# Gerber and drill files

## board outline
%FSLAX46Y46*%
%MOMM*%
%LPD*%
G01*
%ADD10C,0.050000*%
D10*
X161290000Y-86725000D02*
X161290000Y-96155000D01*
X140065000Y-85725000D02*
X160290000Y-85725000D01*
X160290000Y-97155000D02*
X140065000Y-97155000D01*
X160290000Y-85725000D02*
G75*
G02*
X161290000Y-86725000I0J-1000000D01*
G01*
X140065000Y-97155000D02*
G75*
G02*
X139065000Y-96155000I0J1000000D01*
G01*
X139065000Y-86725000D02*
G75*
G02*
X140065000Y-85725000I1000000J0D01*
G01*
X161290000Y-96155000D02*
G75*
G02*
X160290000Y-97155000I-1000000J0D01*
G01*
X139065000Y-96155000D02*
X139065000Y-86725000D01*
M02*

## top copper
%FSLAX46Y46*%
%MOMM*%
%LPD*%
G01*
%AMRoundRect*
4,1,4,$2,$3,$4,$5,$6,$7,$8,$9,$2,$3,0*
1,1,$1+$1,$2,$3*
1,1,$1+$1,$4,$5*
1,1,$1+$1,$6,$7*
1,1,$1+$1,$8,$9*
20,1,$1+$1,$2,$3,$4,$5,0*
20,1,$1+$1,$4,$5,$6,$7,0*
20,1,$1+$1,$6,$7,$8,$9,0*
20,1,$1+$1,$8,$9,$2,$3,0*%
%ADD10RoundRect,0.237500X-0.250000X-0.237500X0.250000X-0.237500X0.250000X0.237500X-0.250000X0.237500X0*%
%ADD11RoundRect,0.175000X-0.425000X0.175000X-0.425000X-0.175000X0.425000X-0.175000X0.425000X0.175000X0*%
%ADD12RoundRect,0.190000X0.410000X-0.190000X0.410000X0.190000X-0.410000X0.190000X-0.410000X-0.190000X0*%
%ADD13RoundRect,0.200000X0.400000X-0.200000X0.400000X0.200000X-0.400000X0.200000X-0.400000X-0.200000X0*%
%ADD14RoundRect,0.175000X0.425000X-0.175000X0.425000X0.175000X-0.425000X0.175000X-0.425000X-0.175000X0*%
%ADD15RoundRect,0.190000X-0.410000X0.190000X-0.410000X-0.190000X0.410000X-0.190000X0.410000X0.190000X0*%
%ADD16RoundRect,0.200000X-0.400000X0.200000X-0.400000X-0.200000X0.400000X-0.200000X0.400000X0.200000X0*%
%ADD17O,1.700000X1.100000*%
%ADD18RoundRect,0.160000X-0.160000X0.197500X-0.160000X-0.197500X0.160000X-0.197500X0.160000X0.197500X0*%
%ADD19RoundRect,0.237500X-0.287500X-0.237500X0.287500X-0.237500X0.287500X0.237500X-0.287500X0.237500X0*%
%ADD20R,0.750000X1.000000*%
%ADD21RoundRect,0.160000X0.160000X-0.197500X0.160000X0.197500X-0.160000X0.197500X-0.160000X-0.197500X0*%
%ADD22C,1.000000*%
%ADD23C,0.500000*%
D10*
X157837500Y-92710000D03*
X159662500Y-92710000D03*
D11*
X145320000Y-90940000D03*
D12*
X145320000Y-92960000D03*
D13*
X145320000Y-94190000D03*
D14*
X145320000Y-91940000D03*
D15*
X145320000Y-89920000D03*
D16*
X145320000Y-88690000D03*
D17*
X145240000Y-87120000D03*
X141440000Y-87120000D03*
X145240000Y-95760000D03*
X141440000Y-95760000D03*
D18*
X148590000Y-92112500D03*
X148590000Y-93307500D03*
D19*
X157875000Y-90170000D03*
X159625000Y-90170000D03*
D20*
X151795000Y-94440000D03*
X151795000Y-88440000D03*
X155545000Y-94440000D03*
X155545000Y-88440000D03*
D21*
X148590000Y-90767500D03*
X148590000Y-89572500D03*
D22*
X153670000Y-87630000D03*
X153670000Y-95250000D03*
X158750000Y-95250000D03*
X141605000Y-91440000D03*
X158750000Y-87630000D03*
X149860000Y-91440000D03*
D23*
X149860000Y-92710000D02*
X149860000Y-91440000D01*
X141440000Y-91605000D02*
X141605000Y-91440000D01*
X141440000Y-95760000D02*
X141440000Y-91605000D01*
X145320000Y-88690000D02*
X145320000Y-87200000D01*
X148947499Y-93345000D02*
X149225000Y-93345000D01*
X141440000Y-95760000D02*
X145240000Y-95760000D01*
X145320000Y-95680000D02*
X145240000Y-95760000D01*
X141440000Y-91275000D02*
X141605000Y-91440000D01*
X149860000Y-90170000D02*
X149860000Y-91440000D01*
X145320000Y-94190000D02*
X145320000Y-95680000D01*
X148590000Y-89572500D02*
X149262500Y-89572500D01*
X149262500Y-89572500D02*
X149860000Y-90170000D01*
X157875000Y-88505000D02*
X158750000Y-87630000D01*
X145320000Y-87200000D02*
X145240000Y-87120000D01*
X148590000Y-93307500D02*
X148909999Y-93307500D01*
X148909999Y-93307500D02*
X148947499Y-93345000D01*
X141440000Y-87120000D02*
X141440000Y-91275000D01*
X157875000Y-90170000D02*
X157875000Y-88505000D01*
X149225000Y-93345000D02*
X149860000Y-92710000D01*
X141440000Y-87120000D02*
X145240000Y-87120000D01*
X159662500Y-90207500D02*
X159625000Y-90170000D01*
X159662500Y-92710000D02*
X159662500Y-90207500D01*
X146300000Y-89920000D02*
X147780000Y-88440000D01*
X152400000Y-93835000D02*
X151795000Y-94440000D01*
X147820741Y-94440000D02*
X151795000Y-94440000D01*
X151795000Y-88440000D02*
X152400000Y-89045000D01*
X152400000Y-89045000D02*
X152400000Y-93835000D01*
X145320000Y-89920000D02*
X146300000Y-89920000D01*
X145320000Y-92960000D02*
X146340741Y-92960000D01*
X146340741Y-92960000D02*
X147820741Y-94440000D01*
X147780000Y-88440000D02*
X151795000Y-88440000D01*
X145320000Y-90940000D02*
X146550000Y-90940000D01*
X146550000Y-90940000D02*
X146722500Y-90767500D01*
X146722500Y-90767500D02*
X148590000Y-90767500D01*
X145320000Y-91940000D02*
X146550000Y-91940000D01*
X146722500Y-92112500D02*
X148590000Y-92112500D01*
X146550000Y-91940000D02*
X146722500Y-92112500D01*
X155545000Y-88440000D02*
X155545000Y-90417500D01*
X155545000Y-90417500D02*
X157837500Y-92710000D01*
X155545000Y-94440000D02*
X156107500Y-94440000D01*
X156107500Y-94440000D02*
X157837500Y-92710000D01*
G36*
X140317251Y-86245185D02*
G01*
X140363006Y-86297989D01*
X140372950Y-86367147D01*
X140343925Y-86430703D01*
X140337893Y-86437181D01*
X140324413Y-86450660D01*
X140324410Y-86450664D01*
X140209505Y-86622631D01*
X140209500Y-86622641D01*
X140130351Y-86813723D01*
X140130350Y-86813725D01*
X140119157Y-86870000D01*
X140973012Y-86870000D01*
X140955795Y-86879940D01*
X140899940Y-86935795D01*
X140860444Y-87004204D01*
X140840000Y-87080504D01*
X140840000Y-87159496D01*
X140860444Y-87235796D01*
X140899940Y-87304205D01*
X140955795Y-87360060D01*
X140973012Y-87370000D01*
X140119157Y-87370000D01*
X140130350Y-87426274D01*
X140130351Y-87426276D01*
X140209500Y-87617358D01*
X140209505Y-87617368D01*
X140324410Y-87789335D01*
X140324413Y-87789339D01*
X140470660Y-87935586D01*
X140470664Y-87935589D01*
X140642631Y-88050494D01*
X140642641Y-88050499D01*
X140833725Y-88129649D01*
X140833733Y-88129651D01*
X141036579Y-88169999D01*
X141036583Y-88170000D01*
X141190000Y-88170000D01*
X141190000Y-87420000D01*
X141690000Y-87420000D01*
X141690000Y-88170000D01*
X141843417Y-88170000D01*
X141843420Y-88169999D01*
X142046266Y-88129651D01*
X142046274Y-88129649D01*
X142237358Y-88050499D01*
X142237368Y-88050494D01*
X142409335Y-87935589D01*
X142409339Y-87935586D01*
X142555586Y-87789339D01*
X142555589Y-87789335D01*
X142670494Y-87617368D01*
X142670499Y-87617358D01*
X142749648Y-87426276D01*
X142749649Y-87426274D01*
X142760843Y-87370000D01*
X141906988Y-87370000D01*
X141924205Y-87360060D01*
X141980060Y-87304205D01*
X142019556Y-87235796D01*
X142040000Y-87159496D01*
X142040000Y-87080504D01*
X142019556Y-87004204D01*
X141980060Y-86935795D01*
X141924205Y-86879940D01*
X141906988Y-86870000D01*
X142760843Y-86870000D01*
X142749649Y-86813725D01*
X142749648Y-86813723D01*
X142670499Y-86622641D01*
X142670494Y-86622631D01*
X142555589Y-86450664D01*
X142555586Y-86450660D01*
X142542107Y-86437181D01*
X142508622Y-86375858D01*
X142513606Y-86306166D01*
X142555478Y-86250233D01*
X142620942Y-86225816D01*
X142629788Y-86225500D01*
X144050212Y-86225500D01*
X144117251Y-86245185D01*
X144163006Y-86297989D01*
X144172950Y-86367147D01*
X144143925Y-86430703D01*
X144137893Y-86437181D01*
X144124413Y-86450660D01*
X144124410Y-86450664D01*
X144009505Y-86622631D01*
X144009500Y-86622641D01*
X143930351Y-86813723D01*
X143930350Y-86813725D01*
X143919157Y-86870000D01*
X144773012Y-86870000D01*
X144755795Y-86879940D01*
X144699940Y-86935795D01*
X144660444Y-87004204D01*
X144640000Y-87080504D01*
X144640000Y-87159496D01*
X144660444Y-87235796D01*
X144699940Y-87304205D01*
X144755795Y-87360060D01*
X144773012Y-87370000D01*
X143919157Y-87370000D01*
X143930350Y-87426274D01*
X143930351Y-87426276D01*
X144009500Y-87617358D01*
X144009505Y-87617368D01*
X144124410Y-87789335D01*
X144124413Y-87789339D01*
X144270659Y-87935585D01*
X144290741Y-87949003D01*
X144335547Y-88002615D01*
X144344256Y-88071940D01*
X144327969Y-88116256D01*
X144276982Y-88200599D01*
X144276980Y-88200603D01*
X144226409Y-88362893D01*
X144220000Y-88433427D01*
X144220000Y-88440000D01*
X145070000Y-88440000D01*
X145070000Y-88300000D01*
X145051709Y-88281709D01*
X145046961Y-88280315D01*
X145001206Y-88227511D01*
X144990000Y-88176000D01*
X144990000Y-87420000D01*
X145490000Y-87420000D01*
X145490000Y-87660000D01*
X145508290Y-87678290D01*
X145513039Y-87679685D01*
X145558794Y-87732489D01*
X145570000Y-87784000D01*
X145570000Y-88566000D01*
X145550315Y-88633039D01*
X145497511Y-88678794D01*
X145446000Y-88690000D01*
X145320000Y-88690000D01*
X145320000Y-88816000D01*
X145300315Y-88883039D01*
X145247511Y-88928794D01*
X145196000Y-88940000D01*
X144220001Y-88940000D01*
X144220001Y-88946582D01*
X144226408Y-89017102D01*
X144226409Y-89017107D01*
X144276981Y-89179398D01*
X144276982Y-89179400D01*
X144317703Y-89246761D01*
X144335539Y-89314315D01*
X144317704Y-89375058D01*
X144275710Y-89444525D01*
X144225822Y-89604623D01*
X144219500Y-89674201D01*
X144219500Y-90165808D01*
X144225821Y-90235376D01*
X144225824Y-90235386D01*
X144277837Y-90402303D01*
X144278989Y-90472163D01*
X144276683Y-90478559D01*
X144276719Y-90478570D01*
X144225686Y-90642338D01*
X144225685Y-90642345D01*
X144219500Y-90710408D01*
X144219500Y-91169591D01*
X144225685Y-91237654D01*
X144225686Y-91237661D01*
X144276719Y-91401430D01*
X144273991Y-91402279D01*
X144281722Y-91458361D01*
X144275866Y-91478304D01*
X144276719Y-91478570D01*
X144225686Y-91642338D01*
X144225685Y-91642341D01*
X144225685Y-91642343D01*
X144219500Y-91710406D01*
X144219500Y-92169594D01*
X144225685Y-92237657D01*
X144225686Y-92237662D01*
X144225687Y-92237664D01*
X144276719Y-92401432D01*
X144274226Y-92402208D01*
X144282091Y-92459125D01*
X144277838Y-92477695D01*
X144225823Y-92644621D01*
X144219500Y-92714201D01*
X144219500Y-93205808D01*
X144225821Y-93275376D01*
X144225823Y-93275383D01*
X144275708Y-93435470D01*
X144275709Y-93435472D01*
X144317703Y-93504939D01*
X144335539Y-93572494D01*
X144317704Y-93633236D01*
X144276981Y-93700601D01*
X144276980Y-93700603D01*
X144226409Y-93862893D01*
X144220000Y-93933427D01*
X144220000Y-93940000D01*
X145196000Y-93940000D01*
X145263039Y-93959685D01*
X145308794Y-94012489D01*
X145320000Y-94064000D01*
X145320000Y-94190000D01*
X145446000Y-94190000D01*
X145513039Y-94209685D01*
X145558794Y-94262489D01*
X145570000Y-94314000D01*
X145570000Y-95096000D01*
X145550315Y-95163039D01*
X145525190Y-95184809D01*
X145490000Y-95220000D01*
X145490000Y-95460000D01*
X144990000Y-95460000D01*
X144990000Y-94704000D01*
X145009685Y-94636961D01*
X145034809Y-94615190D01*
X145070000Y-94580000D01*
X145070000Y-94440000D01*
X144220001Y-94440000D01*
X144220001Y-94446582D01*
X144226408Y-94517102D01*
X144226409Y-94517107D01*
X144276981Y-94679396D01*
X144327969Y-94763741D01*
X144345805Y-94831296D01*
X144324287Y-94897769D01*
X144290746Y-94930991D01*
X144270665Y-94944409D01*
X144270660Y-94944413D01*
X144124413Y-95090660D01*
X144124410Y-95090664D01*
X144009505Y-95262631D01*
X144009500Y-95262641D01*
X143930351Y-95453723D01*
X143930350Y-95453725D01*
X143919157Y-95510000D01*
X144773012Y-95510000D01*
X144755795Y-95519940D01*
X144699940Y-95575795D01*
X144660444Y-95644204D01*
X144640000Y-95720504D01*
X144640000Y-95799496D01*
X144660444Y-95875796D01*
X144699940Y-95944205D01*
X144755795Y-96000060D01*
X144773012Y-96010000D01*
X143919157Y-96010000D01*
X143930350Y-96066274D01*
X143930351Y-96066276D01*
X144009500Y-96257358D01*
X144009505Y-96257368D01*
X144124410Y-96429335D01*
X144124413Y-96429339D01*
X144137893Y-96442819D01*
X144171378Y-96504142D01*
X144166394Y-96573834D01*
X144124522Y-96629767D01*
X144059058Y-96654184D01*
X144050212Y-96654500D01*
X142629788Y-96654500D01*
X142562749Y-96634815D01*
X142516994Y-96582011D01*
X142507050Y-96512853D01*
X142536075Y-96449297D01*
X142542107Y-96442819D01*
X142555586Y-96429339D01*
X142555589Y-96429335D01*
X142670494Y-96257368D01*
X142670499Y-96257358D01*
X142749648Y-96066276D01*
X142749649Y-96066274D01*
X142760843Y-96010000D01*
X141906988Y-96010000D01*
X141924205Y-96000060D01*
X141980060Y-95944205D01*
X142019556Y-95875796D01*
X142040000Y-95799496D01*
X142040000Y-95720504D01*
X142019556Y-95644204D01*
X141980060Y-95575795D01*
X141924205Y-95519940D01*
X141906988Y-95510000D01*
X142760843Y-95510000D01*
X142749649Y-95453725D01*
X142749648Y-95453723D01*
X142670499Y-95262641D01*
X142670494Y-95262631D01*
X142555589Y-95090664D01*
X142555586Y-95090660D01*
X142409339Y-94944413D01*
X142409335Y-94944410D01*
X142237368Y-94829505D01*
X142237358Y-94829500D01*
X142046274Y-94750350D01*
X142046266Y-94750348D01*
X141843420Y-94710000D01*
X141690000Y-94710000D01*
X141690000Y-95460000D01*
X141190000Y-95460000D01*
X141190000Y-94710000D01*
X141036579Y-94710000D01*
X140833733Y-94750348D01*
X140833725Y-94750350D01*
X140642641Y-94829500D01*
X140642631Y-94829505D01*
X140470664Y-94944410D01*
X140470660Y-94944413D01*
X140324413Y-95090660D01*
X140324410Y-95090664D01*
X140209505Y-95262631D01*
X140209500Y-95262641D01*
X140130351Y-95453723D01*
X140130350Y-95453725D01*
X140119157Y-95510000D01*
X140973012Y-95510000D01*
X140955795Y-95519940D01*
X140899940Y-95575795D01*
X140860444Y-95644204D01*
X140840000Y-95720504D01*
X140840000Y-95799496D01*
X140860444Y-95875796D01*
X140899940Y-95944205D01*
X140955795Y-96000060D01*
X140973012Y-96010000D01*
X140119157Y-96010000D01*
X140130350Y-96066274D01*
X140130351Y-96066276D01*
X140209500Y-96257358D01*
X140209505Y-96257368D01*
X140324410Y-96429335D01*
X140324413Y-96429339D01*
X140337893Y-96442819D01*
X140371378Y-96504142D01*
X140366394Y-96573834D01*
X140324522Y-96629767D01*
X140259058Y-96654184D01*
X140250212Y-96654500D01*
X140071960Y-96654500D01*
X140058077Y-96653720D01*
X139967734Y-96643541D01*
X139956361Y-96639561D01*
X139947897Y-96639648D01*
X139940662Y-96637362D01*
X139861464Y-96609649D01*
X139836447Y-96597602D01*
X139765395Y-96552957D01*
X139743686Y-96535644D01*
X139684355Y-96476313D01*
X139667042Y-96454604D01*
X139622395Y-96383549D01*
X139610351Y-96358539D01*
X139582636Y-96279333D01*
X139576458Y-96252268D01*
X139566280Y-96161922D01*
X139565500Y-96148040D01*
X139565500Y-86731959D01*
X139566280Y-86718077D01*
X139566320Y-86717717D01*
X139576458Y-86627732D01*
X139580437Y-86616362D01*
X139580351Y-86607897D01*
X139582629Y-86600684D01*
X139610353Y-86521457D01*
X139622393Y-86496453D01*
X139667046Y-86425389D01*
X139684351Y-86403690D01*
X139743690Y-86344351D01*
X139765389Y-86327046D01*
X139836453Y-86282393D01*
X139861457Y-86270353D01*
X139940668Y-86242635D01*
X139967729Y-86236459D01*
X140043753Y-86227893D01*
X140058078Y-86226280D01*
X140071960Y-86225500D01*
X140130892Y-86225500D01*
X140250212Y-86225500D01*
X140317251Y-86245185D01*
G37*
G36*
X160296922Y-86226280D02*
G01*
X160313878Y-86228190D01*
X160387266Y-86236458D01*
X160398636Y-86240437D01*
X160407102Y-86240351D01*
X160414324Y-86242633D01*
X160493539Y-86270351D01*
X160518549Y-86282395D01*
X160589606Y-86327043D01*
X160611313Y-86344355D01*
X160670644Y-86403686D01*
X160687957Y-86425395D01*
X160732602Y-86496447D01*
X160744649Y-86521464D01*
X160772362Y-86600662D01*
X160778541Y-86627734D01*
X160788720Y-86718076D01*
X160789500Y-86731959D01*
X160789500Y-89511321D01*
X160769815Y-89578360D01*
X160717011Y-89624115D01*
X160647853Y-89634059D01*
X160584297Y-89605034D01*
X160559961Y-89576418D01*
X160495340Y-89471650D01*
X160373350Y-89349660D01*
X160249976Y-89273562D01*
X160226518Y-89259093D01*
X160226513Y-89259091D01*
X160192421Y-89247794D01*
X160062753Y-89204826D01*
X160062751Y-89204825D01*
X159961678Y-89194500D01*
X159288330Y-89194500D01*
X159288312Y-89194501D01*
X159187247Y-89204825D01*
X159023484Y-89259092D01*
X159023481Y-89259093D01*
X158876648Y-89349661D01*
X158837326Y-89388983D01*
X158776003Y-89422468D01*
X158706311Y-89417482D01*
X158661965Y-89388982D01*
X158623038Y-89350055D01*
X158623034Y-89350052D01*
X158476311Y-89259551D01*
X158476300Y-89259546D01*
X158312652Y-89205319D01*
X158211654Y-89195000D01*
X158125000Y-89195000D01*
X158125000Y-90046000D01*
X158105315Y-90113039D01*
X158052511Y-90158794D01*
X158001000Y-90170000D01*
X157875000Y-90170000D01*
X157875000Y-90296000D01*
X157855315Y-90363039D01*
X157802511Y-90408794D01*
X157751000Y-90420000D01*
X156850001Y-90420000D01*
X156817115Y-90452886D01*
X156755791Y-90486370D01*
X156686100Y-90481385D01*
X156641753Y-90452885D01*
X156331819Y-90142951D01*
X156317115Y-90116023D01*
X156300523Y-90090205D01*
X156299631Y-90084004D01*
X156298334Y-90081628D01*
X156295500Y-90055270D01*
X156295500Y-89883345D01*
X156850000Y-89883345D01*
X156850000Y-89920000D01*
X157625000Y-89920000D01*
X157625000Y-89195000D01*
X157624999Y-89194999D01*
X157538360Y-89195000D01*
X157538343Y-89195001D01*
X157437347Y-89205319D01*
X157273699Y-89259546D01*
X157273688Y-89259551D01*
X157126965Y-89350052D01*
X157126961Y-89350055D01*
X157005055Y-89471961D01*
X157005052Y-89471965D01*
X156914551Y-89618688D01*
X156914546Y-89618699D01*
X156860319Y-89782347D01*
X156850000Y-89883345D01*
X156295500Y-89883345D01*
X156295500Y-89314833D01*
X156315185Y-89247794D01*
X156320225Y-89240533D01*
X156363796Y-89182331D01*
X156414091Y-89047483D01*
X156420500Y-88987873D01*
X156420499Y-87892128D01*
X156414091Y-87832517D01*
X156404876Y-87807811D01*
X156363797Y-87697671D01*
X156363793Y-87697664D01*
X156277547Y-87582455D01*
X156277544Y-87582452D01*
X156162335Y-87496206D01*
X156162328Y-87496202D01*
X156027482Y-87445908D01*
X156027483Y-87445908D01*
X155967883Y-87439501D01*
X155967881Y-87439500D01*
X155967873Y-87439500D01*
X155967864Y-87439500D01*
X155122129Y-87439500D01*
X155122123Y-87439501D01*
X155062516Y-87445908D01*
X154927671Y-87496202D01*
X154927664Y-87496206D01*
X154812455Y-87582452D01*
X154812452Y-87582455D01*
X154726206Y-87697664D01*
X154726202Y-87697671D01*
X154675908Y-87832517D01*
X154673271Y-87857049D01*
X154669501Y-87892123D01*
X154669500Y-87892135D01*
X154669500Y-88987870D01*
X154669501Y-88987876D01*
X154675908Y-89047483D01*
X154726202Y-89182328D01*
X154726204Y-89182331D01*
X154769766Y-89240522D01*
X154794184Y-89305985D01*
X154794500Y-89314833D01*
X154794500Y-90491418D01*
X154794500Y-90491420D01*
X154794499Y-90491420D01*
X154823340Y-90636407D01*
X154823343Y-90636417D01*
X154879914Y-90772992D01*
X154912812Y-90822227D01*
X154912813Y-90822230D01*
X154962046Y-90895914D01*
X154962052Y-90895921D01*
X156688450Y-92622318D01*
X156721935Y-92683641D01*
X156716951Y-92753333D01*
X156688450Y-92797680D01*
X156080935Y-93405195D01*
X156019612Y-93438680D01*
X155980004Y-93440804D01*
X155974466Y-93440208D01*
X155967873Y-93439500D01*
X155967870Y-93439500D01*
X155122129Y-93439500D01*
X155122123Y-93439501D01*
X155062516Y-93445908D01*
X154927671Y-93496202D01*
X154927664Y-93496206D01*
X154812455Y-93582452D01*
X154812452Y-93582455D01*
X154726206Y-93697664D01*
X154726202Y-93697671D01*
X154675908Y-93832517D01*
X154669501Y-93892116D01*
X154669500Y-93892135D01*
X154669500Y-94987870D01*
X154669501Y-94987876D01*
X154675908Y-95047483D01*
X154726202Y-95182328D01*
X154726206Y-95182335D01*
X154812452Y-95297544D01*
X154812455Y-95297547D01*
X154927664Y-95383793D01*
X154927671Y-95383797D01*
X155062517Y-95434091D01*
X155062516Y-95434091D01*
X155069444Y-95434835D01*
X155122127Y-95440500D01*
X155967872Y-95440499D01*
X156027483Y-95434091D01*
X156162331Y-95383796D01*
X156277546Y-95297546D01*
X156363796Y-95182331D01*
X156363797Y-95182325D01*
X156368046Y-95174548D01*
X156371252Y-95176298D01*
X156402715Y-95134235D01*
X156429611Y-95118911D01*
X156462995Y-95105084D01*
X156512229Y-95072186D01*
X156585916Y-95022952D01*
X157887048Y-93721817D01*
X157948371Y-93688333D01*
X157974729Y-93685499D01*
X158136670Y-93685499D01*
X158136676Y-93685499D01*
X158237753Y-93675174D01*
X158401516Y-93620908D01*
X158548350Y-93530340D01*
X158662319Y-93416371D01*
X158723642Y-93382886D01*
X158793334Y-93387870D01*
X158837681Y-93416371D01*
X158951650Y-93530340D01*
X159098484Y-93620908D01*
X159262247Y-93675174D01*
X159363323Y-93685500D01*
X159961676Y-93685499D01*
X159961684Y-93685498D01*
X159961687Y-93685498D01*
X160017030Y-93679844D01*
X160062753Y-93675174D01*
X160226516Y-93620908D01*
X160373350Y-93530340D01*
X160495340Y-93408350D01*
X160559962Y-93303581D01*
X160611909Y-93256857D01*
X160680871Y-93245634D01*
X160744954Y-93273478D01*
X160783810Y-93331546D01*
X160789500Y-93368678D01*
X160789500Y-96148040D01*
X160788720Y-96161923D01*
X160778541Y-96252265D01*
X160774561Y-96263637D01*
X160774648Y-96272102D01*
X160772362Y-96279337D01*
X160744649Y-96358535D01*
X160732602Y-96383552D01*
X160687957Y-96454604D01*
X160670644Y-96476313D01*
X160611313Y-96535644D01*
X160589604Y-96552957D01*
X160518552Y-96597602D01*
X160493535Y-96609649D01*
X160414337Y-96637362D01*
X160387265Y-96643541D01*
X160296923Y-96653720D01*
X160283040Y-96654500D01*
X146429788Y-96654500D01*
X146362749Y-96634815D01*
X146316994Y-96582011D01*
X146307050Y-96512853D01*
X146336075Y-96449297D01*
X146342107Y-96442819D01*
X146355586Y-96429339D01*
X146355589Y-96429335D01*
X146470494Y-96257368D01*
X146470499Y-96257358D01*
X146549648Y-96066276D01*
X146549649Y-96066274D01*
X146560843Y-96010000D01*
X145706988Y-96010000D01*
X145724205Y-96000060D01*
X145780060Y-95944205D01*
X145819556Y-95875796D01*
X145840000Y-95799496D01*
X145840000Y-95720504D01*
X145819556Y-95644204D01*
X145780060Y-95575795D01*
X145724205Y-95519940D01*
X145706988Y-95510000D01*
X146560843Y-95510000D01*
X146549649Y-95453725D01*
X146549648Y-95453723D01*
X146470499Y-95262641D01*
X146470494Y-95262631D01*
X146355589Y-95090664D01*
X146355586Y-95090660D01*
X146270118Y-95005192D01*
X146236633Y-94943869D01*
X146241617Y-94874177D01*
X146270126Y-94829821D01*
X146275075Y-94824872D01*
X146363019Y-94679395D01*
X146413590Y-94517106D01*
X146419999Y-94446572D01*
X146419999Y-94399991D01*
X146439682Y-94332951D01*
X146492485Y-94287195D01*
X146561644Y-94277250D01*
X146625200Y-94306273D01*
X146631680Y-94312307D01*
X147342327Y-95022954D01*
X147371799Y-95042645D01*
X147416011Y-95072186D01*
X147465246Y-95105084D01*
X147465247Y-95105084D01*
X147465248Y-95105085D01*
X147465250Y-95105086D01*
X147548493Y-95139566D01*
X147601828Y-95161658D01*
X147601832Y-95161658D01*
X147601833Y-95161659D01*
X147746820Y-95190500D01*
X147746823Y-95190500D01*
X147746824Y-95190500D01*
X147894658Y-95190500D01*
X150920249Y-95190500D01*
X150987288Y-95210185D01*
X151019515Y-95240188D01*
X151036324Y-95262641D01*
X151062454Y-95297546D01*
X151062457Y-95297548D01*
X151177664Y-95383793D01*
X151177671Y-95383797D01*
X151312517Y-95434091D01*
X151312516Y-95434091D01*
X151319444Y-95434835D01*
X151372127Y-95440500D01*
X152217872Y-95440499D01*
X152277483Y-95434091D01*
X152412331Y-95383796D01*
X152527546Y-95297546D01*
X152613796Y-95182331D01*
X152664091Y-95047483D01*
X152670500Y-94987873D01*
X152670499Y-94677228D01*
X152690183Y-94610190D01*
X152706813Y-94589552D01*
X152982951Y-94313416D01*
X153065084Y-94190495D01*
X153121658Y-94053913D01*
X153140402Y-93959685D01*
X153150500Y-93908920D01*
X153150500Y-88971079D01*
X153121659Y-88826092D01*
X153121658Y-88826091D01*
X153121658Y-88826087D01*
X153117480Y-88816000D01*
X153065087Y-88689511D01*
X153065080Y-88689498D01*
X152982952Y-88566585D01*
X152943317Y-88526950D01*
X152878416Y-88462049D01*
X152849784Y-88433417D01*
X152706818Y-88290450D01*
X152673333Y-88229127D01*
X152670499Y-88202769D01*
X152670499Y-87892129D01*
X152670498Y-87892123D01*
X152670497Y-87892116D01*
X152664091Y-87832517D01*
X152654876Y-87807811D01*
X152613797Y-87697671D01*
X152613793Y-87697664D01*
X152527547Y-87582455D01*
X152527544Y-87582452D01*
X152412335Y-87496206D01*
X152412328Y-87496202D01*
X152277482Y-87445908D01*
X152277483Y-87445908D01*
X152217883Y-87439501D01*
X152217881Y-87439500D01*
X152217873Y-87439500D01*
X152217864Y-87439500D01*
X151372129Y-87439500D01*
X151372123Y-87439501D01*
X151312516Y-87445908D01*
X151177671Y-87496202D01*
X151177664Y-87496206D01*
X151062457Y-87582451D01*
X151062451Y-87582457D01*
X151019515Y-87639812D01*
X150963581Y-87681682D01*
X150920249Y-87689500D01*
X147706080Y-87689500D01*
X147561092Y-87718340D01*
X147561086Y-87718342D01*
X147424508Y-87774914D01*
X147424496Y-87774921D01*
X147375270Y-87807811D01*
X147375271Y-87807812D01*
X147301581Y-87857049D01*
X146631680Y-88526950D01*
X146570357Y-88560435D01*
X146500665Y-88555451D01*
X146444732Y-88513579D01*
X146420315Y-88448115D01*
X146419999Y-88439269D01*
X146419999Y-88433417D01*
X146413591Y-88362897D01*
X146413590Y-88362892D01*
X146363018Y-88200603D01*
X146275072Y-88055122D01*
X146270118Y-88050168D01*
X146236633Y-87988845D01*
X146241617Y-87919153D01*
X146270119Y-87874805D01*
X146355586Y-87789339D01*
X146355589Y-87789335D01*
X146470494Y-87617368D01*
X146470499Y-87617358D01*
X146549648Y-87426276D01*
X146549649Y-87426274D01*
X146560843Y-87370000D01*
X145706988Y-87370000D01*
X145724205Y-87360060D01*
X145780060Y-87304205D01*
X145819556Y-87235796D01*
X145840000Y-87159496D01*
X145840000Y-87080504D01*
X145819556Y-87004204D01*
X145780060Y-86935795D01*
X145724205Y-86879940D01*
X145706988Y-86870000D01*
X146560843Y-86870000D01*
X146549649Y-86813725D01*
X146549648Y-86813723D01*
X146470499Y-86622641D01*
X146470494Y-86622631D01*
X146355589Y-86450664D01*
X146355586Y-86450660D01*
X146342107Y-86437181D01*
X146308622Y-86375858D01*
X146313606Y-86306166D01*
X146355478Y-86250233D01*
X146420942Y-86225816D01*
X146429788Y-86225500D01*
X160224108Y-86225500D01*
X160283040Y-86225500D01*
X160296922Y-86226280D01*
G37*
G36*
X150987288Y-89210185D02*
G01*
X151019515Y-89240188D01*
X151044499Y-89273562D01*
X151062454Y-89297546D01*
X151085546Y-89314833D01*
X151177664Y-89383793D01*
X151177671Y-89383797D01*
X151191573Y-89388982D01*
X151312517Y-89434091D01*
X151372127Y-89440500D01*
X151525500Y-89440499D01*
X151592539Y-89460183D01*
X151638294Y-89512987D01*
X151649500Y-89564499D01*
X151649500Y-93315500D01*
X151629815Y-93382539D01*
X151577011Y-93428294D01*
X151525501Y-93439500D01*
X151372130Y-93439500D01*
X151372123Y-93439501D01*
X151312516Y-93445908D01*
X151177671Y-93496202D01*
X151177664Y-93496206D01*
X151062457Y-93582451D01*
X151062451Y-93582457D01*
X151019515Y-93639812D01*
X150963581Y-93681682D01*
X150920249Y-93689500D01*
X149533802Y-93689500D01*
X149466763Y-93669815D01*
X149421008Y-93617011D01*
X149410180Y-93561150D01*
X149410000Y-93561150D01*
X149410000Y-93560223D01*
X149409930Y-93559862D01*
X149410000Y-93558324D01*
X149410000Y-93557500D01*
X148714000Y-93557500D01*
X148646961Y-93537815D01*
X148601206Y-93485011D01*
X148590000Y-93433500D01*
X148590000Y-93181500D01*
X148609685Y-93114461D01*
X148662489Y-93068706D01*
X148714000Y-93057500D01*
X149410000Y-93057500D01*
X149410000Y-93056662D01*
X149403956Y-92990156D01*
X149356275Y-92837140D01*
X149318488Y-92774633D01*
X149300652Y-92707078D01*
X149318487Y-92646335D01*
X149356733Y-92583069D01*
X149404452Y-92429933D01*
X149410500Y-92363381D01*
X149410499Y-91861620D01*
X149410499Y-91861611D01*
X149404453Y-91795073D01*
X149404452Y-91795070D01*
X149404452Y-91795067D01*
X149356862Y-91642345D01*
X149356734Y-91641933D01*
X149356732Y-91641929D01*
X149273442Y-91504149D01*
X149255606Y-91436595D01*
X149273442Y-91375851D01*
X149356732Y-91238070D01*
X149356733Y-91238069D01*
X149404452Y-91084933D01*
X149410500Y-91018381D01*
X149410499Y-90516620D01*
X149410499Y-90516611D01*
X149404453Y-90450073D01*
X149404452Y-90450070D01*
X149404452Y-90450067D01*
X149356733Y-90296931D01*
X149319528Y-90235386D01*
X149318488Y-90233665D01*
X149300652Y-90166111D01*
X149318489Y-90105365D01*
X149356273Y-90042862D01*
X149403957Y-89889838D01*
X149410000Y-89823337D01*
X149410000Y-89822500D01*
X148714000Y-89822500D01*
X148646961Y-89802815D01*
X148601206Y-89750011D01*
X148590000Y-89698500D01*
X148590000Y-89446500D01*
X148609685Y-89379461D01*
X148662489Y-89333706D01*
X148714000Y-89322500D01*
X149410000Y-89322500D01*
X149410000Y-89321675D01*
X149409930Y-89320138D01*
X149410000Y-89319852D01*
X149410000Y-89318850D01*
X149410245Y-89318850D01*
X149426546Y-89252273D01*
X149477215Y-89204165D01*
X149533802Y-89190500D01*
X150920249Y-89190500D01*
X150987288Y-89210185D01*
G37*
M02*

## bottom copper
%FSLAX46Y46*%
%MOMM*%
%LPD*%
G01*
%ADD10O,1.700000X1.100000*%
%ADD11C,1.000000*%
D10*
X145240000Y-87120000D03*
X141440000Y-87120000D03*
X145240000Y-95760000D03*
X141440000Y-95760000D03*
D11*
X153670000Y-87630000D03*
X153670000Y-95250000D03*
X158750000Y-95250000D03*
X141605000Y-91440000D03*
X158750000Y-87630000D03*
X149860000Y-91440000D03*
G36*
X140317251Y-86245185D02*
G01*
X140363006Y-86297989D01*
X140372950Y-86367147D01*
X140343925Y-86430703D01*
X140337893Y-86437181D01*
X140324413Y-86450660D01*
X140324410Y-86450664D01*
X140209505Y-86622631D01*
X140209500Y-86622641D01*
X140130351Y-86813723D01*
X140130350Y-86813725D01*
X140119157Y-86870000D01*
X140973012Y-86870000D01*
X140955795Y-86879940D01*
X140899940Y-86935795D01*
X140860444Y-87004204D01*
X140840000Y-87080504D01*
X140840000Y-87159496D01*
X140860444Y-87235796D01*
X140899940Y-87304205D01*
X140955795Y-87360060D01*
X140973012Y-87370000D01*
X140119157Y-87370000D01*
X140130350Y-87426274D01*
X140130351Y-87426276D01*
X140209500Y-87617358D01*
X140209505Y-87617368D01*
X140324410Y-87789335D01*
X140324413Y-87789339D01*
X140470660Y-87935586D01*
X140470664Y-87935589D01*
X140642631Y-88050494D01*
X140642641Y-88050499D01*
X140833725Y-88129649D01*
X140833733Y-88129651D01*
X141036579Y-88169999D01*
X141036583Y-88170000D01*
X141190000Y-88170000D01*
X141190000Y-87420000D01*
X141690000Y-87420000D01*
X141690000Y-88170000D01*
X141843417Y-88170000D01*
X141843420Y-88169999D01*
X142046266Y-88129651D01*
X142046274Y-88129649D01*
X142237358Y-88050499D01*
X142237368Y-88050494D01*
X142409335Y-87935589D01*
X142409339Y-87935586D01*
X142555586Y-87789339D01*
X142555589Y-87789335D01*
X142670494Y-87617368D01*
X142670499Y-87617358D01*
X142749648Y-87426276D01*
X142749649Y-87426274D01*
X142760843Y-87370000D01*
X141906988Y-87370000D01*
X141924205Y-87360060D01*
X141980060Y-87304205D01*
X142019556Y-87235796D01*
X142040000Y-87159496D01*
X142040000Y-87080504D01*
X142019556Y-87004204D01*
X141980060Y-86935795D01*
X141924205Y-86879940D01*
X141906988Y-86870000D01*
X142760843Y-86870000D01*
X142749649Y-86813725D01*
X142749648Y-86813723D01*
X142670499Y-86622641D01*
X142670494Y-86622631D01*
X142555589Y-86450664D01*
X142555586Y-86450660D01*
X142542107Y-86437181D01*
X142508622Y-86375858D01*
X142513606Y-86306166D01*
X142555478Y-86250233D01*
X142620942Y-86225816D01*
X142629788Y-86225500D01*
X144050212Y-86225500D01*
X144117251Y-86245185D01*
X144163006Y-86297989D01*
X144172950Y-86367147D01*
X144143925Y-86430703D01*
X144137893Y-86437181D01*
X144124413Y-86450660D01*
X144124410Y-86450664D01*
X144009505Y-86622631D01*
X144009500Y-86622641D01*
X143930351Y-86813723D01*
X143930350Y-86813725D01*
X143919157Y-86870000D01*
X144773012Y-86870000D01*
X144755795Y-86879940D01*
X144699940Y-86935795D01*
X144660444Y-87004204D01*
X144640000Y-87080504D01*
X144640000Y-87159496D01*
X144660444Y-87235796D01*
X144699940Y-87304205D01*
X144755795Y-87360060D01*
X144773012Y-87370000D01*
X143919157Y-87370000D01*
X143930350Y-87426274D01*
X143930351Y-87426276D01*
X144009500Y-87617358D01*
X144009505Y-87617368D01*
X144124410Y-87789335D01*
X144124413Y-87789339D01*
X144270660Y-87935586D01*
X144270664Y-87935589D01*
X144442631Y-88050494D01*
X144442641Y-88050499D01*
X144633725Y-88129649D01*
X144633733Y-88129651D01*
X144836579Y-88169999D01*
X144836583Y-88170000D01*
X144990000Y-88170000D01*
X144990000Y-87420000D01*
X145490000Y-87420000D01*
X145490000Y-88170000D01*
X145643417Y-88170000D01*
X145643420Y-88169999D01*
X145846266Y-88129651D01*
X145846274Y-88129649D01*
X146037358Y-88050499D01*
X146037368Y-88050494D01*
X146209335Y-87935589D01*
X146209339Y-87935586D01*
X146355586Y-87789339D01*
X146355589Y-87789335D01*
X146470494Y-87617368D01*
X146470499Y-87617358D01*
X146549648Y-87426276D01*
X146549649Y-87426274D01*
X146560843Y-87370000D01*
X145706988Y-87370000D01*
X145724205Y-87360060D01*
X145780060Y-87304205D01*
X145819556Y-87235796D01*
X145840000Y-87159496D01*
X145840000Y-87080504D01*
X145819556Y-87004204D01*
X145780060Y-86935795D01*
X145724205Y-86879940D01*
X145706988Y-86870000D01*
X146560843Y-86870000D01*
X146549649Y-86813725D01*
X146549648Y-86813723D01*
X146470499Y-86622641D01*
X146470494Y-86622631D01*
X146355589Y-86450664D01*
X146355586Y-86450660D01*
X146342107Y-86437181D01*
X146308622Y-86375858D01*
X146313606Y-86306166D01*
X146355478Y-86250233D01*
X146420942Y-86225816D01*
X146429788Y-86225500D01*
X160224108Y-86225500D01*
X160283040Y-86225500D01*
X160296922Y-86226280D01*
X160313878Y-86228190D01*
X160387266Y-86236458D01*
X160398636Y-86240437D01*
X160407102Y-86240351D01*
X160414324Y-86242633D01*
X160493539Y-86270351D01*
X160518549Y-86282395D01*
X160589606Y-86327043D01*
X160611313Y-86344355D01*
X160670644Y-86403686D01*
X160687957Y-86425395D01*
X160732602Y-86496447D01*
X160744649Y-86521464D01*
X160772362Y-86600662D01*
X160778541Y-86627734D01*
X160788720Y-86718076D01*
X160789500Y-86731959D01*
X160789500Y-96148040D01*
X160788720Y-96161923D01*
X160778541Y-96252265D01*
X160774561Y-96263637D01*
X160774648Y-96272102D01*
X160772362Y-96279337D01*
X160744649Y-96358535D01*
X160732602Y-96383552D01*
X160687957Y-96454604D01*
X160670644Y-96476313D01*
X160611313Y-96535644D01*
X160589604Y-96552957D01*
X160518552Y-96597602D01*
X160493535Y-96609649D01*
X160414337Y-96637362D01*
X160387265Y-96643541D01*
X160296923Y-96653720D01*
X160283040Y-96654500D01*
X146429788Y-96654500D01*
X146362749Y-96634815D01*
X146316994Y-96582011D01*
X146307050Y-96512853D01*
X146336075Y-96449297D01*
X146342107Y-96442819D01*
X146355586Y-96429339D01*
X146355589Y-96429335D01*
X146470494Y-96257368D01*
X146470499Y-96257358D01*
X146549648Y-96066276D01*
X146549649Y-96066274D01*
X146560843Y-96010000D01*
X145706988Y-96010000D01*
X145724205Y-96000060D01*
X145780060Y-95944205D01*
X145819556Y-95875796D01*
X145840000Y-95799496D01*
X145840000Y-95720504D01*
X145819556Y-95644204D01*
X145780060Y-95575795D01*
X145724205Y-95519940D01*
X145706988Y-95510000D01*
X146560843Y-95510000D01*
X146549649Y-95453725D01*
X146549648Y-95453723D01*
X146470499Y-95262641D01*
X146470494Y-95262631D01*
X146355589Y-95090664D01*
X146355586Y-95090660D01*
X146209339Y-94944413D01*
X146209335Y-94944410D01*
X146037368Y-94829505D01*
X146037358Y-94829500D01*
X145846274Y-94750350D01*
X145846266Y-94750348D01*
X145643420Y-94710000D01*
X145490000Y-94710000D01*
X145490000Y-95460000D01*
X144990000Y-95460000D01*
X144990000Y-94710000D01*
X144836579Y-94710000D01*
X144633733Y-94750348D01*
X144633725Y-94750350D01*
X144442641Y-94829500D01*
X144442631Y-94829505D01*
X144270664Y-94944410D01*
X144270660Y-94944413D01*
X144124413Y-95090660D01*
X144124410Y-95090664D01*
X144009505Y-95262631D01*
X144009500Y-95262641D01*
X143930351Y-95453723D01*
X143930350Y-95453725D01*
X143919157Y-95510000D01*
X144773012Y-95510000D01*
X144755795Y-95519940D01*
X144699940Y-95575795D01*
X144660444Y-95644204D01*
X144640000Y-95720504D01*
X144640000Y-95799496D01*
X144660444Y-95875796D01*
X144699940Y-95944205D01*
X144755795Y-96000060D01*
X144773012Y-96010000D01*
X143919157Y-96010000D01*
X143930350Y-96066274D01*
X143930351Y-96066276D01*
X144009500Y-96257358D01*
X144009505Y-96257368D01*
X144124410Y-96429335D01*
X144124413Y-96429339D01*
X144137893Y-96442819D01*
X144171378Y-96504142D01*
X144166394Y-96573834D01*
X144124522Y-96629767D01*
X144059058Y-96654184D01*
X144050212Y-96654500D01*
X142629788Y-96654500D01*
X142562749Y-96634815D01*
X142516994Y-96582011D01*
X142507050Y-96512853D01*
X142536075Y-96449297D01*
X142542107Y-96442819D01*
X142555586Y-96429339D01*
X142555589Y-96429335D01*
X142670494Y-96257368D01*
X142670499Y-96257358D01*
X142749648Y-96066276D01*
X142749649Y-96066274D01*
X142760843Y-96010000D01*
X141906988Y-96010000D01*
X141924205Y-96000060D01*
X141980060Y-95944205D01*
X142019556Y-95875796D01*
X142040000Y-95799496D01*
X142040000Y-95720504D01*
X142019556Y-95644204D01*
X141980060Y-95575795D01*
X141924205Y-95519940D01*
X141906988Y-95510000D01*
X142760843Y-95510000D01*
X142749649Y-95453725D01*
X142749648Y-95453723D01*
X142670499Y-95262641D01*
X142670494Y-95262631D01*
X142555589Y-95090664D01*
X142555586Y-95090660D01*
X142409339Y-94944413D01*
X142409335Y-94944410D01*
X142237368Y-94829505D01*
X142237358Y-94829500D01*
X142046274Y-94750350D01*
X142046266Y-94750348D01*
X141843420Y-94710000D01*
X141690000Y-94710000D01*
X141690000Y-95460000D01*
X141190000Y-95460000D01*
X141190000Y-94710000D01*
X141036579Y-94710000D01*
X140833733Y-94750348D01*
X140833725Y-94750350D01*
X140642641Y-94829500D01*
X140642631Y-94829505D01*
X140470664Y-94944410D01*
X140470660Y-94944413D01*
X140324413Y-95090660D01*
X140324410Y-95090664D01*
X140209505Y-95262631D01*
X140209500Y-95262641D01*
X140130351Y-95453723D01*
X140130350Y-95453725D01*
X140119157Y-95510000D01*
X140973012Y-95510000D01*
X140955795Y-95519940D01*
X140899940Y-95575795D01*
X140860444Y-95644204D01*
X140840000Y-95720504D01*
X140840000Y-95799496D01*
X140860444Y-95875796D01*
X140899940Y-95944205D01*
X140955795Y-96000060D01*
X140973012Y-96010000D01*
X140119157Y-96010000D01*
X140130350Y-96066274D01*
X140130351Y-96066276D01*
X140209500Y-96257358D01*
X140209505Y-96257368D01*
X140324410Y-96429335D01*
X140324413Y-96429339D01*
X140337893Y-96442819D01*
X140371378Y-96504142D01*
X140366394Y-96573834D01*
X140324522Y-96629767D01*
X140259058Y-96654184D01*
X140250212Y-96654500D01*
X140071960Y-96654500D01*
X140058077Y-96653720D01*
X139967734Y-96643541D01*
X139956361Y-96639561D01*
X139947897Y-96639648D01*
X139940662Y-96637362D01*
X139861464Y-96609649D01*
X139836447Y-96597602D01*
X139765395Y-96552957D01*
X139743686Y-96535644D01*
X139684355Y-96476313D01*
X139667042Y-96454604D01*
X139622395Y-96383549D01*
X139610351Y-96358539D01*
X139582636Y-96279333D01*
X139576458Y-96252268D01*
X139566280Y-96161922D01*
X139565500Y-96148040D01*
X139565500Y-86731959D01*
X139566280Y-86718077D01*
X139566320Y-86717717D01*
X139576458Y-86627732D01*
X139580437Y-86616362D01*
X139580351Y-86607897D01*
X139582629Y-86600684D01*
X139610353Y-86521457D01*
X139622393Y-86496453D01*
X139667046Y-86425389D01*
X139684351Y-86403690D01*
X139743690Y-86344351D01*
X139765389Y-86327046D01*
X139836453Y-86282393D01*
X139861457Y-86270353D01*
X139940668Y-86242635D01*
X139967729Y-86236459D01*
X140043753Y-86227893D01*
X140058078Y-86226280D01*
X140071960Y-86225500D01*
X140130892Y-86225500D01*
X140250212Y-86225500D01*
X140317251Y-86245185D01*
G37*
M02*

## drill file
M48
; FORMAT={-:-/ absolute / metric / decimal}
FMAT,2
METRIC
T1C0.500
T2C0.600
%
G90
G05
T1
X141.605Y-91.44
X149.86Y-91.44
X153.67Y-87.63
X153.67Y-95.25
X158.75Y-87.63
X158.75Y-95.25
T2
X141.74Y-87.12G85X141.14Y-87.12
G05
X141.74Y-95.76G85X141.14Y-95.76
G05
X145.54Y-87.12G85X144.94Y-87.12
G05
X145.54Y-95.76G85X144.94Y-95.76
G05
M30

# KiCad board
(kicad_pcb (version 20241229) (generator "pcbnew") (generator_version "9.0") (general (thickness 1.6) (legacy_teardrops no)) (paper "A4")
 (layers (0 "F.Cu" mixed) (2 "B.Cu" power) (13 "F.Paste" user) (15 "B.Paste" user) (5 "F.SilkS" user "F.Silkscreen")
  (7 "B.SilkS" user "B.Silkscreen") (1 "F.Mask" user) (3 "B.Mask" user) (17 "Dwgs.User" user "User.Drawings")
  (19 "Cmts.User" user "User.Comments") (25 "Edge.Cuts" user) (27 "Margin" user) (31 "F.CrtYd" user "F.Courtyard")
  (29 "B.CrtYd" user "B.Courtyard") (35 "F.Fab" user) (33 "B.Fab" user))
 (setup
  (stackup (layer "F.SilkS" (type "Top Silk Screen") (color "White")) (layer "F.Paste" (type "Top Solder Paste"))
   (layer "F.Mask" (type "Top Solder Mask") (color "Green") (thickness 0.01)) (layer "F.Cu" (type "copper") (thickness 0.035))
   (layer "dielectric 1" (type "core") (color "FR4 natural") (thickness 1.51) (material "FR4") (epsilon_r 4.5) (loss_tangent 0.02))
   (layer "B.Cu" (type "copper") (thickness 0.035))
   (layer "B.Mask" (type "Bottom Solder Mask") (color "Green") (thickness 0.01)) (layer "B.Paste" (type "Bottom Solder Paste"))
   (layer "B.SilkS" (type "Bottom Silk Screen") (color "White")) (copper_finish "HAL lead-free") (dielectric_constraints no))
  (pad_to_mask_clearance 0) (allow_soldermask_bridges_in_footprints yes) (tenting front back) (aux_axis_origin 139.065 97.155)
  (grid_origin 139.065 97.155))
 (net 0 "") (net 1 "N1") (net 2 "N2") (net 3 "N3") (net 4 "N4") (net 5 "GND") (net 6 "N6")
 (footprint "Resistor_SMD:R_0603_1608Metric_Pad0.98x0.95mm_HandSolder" (layer "F.Cu") (at 158.75 92.71)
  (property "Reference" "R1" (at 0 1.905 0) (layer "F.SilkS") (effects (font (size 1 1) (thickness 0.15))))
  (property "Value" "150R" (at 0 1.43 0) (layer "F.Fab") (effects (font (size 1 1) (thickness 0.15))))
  (pad "1" smd roundrect (at -0.9125 0) (size 0.975 0.95) (layers "F.Cu" "F.Mask" "F.Paste") (roundrect_rratio 0.25) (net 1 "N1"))
  (pad "2" smd roundrect (at 0.9125 0) (size 0.975 0.95) (layers "F.Cu" "F.Mask" "F.Paste") (roundrect_rratio 0.25) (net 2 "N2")))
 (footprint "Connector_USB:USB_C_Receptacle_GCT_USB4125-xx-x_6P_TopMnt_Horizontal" (layer "F.Cu") (at 142.24 91.44 -90)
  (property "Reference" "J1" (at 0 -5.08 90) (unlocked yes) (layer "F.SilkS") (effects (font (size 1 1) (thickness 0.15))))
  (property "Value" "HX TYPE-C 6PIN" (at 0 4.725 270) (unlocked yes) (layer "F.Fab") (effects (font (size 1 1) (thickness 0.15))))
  (pad "A5" smd roundrect (at -0.5 -3.08 270) (size 0.7 1.2) (layers "F.Cu" "F.Mask" "F.Paste") (roundrect_rratio 0.25) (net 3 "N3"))
  (pad "A9" smd roundrect (at 1.52 -3.08 90) (size 0.76 1.2) (layers "F.Cu" "F.Mask" "F.Paste") (roundrect_rratio 0.25) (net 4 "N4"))
  (pad "A12" smd roundrect (at 2.75 -3.08 90) (size 0.8 1.2) (layers "F.Cu" "F.Mask" "F.Paste") (roundrect_rratio 0.25) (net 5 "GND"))
  (pad "B5" smd roundrect (at 0.5 -3.08 90) (size 0.7 1.2) (layers "F.Cu" "F.Mask" "F.Paste") (roundrect_rratio 0.25) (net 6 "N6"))
  (pad "B9" smd roundrect (at -1.52 -3.08 270) (size 0.76 1.2) (layers "F.Cu" "F.Mask" "F.Paste") (roundrect_rratio 0.25) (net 4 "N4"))
  (pad "B12" smd roundrect (at -2.75 -3.08 270) (size 0.8 1.2) (layers "F.Cu" "F.Mask" "F.Paste") (roundrect_rratio 0.25) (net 5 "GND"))
  (pad "S1" thru_hole oval (at -4.32 -3 270) (size 1.1 1.7) (drill oval 0.6 1.2) (layers "*.Cu" "*.Mask" "F.Paste")
   (remove_unused_layers no) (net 5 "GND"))
  (pad "S1" thru_hole oval (at -4.32 0.8 270) (size 1.1 1.7) (drill oval 0.6 1.2) (layers "*.Cu" "*.Mask" "F.Paste")
   (remove_unused_layers no) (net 5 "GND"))
  (pad "S1" thru_hole oval (at 4.32 -3 270) (size 1.1 1.7) (drill oval 0.6 1.2) (layers "*.Cu" "*.Mask" "F.Paste") (remove_unused_layers no)
   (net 5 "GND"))
  (pad "S1" thru_hole oval (at 4.32 0.8 270) (size 1.1 1.7) (drill oval 0.6 1.2) (layers "*.Cu" "*.Mask" "F.Paste")
   (remove_unused_layers no) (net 5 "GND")))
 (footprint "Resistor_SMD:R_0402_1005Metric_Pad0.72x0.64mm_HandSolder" (layer "F.Cu") (at 148.59 92.71 -90)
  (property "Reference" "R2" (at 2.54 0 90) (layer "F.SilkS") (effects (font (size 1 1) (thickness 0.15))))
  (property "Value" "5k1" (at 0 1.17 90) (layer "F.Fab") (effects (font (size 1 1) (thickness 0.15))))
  (pad "1" smd roundrect (at -0.5975 0 270) (size 0.715 0.64) (layers "F.Cu" "F.Mask" "F.Paste") (roundrect_rratio 0.25) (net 6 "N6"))
  (pad "2" smd roundrect (at 0.5975 0 270) (size 0.715 0.64) (layers "F.Cu" "F.Mask" "F.Paste") (roundrect_rratio 0.25) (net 5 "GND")))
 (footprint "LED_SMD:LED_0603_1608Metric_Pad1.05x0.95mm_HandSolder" (layer "F.Cu") (at 158.75 90.17)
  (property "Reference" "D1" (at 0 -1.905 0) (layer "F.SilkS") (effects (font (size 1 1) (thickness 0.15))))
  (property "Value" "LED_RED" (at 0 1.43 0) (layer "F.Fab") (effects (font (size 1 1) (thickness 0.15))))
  (pad "1" smd roundrect (at -0.875 0) (size 1.05 0.95) (layers "F.Cu" "F.Mask" "F.Paste") (roundrect_rratio 0.25) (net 5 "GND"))
  (pad "2" smd roundrect (at 0.875 0) (size 1.05 0.95) (layers "F.Cu" "F.Mask" "F.Paste") (roundrect_rratio 0.25) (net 2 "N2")))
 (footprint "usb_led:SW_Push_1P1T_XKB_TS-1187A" (layer "F.Cu") (at 153.67 91.44 90)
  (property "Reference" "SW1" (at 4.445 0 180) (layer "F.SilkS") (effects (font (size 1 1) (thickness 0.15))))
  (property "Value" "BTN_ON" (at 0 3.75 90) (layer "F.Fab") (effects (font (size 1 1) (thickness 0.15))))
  (pad "1" smd rect (at -3 -1.875 90) (size 1 0.75) (layers "F.Cu" "F.Mask" "F.Paste") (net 4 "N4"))
  (pad "1" smd rect (at 3 -1.875 90) (size 1 0.75) (layers "F.Cu" "F.Mask" "F.Paste") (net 4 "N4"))
  (pad "2" smd rect (at -3 1.875 90) (size 1 0.75) (layers "F.Cu" "F.Mask" "F.Paste") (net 1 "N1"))
  (pad "2" smd rect (at 3 1.875 90) (size 1 0.75) (layers "F.Cu" "F.Mask" "F.Paste") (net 1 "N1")))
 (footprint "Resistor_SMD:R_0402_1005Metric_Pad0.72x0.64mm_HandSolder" (layer "F.Cu") (at 148.59 90.17 90)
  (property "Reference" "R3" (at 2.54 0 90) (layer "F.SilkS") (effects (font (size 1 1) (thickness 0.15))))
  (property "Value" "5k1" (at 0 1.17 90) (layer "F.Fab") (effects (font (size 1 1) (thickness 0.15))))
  (pad "1" smd roundrect (at -0.5975 0 90) (size 0.715 0.64) (layers "F.Cu" "F.Mask" "F.Paste") (roundrect_rratio 0.25) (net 3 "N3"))
  (pad "2" smd roundrect (at 0.5975 0 90) (size 0.715 0.64) (layers "F.Cu" "F.Mask" "F.Paste") (roundrect_rratio 0.25) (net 5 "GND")))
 (gr_line (start 161.29 86.725) (end 161.29 96.155) (stroke (width 0.05) (type default)) (layer "Edge.Cuts"))
 (gr_line (start 140.065 85.725) (end 160.29 85.725) (stroke (width 0.05) (type default)) (layer "Edge.Cuts"))
 (gr_line (start 160.29 97.155) (end 140.065 97.155) (stroke (width 0.05) (type default)) (layer "Edge.Cuts"))
 (gr_arc (start 160.29 85.725) (mid 160.997107 86.017893) (end 161.29 86.725) (stroke (width 0.05) (type default)) (layer "Edge.Cuts"))
 (gr_arc (start 140.065 97.155) (mid 139.357893 96.862107) (end 139.065 96.155) (stroke (width 0.05) (type default)) (layer "Edge.Cuts"))
 (gr_arc (start 139.065 86.725) (mid 139.357893 86.017893) (end 140.065 85.725) (stroke (width 0.05) (type default)) (layer "Edge.Cuts"))
 (gr_arc (start 161.29 96.155) (mid 160.997107 96.862107) (end 160.29 97.155) (stroke (width 0.05) (type default)) (layer "Edge.Cuts"))
 (gr_line (start 139.065 96.155) (end 139.065 86.725) (stroke (width 0.05) (type default)) (layer "Edge.Cuts"))
 (segment (start 149.86 92.71) (end 149.86 91.44) (width 0.5) (layer "F.Cu") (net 5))
 (segment (start 141.44 91.605) (end 141.605 91.44) (width 0.5) (layer "F.Cu") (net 5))
 (segment (start 141.44 95.76) (end 141.44 91.605) (width 0.5) (layer "F.Cu") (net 5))
 (segment (start 145.32 88.69) (end 145.32 87.2) (width 0.5) (layer "F.Cu") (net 5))
 (segment (start 148.947499 93.345) (end 149.225 93.345) (width 0.5) (layer "F.Cu") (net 5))
 (segment (start 141.44 95.76) (end 145.24 95.76) (width 0.5) (layer "F.Cu") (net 5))
 (segment (start 145.32 95.68) (end 145.24 95.76) (width 0.5) (layer "F.Cu") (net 5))
 (segment (start 141.44 91.275) (end 141.605 91.44) (width 0.5) (layer "F.Cu") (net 5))
 (segment (start 149.86 90.17) (end 149.86 91.44) (width 0.5) (layer "F.Cu") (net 5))
 (segment (start 145.32 94.19) (end 145.32 95.68) (width 0.5) (layer "F.Cu") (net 5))
 (segment (start 148.59 89.5725) (end 149.2625 89.5725) (width 0.5) (layer "F.Cu") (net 5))
 (segment (start 149.2625 89.5725) (end 149.86 90.17) (width 0.5) (layer "F.Cu") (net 5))
 (segment (start 157.875 88.505) (end 158.75 87.63) (width 0.5) (layer "F.Cu") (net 5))
 (segment (start 145.32 87.2) (end 145.24 87.12) (width 0.5) (layer "F.Cu") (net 5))
 (segment (start 148.59 93.3075) (end 148.909999 93.3075) (width 0.5) (layer "F.Cu") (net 5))
 (segment (start 148.909999 93.3075) (end 148.947499 93.345) (width 0.5) (layer "F.Cu") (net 5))
 (segment (start 141.44 87.12) (end 141.44 91.275) (width 0.5) (layer "F.Cu") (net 5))
 (segment (start 157.875 90.17) (end 157.875 88.505) (width 0.5) (layer "F.Cu") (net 5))
 (segment (start 149.225 93.345) (end 149.86 92.71) (width 0.5) (layer "F.Cu") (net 5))
 (segment (start 141.44 87.12) (end 145.24 87.12) (width 0.5) (layer "F.Cu") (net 5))
 (via (at 153.67 87.63) (size 1) (drill 0.5) (layers "F.Cu" "B.Cu") (free yes) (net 5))
 (via (at 153.67 95.25) (size 1) (drill 0.5) (layers "F.Cu" "B.Cu") (free yes) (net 5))
 (via (at 158.75 95.25) (size 1) (drill 0.5) (layers "F.Cu" "B.Cu") (free yes) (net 5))
 (via (at 141.605 91.44) (size 1) (drill 0.5) (layers "F.Cu" "B.Cu") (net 5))
 (via (at 158.75 87.63) (size 1) (drill 0.5) (layers "F.Cu" "B.Cu") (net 5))
 (via (at 149.86 91.44) (size 1) (drill 0.5) (layers "F.Cu" "B.Cu") (free yes) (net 5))
 (segment (start 159.6625 90.2075) (end 159.625 90.17) (width 0.5) (layer "F.Cu") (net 2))
 (segment (start 159.6625 92.71) (end 159.6625 90.2075) (width 0.5) (layer "F.Cu") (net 2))
 (segment (start 146.3 89.92) (end 147.78 88.44) (width 0.5) (layer "F.Cu") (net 4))
 (segment (start 152.4 93.835) (end 151.795 94.44) (width 0.5) (layer "F.Cu") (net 4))
 (segment (start 147.820741 94.44) (end 151.795 94.44) (width 0.5) (layer "F.Cu") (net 4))
 (segment (start 151.795 88.44) (end 152.4 89.045) (width 0.5) (layer "F.Cu") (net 4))
 (segment (start 152.4 89.045) (end 152.4 93.835) (width 0.5) (layer "F.Cu") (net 4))
 (segment (start 145.32 89.92) (end 146.3 89.92) (width 0.5) (layer "F.Cu") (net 4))
 (segment (start 145.32 92.96) (end 146.340741 92.96) (width 0.5) (layer "F.Cu") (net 4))
 (segment (start 146.340741 92.96) (end 147.820741 94.44) (width 0.5) (layer "F.Cu") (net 4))
 (segment (start 147.78 88.44) (end 151.795 88.44) (width 0.5) (layer "F.Cu") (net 4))
 (segment (start 145.32 90.94) (end 146.55 90.94) (width 0.5) (layer "F.Cu") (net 3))
 (segment (start 146.55 90.94) (end 146.7225 90.7675) (width 0.5) (layer "F.Cu") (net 3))
 (segment (start 146.7225 90.7675) (end 148.59 90.7675) (width 0.5) (layer "F.Cu") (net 3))
 (segment (start 145.32 91.94) (end 146.55 91.94) (width 0.5) (layer "F.Cu") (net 6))
 (segment (start 146.7225 92.1125) (end 148.59 92.1125) (width 0.5) (layer "F.Cu") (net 6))
 (segment (start 146.55 91.94) (end 146.7225 92.1125) (width 0.5) (layer "F.Cu") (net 6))
 (segment (start 155.545 88.44) (end 155.545 90.4175) (width 0.5) (layer "F.Cu") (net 1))
 (segment (start 155.545 90.4175) (end 157.8375 92.71) (width 0.5) (layer "F.Cu") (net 1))
 (segment (start 155.545 94.44) (end 156.1075 94.44) (width 0.5) (layer "F.Cu") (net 1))
 (segment (start 156.1075 94.44) (end 157.8375 92.71) (width 0.5) (layer "F.Cu") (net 1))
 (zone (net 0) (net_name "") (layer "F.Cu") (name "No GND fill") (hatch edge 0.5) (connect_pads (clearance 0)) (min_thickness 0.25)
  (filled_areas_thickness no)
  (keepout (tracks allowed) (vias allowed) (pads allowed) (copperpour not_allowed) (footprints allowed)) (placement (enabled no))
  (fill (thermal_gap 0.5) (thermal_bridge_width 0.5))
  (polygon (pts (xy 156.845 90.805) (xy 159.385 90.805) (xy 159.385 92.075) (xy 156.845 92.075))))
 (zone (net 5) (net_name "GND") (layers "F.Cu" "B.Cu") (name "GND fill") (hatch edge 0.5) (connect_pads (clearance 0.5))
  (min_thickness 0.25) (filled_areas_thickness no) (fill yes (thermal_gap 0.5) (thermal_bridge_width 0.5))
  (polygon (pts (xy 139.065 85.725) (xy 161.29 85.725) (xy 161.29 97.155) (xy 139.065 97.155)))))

